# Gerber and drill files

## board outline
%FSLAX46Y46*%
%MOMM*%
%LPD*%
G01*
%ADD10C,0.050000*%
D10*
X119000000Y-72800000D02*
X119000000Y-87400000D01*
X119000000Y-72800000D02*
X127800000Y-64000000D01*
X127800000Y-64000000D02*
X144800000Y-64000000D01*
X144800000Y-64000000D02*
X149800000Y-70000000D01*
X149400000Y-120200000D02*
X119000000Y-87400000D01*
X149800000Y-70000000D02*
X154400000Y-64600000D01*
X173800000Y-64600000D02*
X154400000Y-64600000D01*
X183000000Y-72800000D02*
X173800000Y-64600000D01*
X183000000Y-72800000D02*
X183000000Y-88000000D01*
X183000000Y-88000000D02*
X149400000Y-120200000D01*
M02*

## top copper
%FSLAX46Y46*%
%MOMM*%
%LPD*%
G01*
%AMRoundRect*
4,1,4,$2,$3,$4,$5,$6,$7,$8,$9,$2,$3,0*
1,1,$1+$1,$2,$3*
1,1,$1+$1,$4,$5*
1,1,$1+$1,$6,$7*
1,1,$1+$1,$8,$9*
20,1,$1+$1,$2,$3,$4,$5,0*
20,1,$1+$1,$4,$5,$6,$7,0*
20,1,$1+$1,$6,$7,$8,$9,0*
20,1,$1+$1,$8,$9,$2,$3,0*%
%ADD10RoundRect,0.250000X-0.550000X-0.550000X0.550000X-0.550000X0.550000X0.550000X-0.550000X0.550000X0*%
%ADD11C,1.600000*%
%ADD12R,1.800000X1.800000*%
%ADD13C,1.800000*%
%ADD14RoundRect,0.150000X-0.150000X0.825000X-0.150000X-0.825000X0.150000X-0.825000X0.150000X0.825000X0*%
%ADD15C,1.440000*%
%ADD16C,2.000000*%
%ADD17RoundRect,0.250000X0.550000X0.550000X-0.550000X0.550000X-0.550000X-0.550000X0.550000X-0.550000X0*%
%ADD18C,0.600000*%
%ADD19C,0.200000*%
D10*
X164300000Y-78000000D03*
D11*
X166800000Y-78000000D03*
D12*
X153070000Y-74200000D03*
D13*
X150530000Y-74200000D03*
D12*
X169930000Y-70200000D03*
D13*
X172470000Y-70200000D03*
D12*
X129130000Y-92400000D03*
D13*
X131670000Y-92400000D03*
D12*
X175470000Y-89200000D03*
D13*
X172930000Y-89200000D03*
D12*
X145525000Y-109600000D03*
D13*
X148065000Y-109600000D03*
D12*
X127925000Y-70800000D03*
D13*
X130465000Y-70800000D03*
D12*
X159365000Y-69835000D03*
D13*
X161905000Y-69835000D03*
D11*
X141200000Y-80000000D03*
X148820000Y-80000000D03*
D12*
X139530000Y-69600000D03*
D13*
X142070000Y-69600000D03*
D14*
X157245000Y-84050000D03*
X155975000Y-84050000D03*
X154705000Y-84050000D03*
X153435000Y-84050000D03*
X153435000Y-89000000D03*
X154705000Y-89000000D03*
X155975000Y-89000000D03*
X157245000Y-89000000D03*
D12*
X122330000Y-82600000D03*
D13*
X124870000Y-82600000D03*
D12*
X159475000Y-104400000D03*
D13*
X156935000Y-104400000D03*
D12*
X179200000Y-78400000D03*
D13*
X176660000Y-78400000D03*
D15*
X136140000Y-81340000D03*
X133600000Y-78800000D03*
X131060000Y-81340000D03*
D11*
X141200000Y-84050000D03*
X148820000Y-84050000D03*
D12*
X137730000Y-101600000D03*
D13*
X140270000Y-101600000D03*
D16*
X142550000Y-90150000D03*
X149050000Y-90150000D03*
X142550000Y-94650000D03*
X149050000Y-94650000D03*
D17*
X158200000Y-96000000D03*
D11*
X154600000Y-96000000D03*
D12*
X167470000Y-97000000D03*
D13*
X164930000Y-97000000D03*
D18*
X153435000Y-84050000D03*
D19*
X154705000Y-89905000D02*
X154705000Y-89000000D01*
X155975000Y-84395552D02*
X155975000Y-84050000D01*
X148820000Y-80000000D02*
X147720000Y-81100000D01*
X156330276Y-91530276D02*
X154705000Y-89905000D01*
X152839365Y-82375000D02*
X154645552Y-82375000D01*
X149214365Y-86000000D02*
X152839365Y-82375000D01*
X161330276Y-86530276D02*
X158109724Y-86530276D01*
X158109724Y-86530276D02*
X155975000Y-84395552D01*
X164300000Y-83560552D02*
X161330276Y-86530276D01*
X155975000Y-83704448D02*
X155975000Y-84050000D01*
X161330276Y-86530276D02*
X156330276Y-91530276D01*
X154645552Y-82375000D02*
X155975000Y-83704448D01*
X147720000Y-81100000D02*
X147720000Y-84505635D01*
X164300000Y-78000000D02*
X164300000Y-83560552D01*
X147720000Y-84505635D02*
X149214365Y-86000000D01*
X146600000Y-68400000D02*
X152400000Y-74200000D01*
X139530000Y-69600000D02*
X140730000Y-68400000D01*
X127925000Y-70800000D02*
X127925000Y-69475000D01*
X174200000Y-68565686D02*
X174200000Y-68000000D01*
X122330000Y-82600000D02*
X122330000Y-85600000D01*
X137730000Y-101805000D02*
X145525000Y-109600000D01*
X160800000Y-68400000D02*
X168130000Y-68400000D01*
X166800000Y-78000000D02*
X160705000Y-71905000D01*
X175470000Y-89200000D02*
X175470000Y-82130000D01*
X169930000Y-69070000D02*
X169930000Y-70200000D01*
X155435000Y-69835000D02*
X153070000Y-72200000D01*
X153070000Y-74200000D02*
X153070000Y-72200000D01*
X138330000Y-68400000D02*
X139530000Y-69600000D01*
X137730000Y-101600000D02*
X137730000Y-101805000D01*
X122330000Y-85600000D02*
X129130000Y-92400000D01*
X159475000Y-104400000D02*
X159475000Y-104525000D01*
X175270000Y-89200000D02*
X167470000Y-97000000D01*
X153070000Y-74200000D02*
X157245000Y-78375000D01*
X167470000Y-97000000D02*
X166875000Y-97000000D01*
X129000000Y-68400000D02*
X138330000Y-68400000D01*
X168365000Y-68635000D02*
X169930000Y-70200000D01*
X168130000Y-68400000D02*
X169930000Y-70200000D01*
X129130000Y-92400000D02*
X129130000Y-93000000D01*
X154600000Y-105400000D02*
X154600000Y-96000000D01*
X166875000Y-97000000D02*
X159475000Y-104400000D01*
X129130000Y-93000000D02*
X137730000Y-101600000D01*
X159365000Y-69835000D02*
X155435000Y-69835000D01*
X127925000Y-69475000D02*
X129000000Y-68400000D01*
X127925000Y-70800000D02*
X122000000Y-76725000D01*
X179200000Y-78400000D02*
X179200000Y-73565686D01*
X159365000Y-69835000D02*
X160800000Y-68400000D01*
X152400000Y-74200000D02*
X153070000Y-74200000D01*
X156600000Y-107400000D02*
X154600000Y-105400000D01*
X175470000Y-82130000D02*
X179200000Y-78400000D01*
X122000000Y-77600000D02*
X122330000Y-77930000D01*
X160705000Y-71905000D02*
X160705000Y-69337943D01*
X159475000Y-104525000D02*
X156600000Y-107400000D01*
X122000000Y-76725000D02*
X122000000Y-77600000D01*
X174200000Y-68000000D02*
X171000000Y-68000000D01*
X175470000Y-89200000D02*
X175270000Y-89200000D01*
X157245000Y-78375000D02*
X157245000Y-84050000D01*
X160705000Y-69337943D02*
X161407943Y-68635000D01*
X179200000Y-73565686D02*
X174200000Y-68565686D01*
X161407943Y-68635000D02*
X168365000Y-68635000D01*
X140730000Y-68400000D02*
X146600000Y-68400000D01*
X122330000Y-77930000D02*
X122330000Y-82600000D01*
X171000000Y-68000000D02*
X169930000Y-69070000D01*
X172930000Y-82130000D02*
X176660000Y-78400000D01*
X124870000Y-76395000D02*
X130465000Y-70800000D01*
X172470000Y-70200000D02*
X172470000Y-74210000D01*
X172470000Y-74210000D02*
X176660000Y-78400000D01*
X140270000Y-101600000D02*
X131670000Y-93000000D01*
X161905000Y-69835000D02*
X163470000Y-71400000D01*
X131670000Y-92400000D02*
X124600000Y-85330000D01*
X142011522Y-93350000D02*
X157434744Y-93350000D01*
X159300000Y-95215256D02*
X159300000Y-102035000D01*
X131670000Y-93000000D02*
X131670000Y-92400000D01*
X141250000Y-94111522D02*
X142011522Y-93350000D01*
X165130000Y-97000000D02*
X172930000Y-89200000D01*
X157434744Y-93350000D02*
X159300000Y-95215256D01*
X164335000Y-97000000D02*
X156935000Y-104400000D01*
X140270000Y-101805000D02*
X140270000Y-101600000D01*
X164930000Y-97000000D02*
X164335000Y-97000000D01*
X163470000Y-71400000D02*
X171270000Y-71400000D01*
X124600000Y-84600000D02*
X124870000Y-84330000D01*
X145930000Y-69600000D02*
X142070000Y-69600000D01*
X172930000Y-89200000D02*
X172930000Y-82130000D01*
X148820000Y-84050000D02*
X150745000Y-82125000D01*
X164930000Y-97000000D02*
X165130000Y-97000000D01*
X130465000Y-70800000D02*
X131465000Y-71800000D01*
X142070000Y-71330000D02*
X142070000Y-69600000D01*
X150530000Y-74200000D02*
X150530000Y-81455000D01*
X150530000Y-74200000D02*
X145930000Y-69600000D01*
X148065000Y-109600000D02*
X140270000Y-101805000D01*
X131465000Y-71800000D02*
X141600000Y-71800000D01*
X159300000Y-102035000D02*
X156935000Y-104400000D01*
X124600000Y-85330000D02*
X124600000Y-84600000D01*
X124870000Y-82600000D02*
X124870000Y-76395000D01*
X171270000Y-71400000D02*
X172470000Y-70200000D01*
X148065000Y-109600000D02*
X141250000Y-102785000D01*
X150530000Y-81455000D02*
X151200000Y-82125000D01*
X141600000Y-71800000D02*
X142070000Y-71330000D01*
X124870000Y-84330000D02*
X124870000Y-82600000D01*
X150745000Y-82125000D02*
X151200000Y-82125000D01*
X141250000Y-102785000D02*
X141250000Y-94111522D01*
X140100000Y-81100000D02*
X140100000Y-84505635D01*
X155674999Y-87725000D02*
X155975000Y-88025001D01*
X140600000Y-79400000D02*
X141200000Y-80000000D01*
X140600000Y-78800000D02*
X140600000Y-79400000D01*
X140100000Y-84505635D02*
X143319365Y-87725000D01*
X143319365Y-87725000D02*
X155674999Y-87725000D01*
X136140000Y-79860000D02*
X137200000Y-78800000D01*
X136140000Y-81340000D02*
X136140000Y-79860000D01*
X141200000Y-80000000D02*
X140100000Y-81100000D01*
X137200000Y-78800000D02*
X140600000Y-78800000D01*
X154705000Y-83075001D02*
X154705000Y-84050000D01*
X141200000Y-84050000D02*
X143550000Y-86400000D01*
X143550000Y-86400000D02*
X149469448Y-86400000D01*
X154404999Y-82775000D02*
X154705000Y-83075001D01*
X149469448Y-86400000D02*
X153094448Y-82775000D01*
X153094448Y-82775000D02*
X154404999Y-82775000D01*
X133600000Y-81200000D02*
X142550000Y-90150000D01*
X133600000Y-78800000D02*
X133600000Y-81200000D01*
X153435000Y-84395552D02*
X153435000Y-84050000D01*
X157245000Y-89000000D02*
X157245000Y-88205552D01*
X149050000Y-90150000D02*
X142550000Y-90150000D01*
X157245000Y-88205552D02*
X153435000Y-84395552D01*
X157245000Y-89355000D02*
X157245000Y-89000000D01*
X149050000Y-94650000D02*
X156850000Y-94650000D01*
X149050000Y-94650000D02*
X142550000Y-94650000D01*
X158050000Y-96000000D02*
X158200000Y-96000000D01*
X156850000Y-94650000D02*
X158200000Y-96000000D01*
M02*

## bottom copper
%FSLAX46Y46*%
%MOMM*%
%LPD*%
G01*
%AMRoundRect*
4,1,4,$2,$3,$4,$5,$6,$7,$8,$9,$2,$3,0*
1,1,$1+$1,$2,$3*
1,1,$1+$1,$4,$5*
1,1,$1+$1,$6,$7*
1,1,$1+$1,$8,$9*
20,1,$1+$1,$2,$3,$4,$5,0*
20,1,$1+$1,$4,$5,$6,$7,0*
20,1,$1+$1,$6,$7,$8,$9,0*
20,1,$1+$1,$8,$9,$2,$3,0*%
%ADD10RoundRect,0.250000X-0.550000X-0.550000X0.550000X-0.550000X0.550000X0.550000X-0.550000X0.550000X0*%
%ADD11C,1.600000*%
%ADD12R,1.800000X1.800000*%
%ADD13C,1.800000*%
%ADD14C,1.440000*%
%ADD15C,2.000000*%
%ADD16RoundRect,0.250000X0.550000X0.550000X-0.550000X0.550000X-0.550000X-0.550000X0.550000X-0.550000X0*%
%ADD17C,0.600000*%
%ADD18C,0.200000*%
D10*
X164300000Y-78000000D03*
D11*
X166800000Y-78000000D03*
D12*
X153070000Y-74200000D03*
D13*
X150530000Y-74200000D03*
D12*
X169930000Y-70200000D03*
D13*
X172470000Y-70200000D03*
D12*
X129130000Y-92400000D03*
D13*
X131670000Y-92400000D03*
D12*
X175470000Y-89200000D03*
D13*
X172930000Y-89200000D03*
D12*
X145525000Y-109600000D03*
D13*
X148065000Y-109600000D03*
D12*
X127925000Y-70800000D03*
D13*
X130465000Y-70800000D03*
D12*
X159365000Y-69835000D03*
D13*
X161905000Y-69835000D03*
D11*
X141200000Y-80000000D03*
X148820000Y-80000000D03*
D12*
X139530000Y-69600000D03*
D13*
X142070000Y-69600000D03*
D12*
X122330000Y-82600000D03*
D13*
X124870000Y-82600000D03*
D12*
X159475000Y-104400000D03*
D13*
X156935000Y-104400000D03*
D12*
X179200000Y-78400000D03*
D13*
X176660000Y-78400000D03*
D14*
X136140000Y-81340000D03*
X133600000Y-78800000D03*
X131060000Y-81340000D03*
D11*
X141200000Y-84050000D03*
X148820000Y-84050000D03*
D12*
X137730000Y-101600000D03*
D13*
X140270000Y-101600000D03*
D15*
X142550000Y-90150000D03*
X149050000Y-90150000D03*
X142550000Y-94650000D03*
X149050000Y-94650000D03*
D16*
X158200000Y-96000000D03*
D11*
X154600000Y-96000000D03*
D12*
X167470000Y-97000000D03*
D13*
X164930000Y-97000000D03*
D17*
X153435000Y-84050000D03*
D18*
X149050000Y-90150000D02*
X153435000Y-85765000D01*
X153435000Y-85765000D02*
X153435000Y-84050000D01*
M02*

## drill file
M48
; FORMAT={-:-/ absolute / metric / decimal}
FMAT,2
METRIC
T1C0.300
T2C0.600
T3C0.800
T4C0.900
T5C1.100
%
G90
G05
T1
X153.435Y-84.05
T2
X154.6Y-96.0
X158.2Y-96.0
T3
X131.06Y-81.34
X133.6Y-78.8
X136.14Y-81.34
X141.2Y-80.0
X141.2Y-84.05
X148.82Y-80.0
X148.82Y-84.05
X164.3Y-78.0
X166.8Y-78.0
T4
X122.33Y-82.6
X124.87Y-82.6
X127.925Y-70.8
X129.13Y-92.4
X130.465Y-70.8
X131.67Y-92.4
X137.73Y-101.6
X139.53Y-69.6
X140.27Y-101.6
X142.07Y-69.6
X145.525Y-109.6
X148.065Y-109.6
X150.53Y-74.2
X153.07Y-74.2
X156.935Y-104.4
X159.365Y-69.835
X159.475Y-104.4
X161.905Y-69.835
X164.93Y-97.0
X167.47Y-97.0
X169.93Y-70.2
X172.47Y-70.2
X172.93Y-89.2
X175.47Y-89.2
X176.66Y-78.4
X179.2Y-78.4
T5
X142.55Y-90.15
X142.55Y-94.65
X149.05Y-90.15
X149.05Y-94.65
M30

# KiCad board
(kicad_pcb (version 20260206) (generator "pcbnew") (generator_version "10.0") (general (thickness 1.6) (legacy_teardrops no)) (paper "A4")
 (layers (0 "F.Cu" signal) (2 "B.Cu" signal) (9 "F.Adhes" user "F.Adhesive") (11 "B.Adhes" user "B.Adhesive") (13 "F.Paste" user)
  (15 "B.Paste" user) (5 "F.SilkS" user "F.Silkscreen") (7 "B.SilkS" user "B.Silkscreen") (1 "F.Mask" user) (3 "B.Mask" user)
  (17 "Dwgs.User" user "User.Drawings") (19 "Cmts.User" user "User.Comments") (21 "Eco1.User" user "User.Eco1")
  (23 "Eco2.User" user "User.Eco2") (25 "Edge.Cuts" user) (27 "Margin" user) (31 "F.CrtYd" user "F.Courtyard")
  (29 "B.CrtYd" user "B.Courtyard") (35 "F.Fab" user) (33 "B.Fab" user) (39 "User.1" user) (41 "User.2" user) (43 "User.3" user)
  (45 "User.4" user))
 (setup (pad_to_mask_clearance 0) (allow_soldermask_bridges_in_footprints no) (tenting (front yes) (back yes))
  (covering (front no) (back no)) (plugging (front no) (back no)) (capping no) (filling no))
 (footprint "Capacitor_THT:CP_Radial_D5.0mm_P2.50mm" (layer "F.Cu") (at 164.3 78)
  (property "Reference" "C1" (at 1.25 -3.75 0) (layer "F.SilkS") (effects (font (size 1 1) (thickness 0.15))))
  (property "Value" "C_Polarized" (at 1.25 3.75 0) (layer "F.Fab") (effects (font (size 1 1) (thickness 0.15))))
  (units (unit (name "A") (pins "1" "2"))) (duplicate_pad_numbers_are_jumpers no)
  (pad "1" thru_hole roundrect (at 0 0) (size 1.6 1.6) (drill 0.8) (layers "*.Cu" "*.Mask") (remove_unused_layers no)
   (roundrect_rratio 0.15625) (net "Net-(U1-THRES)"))
  (pad "2" thru_hole circle (at 2.5 0) (size 1.6 1.6) (drill 0.8) (layers "*.Cu" "*.Mask") (remove_unused_layers no) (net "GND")))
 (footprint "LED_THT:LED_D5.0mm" (layer "F.Cu") (at 153.07 74.2 180)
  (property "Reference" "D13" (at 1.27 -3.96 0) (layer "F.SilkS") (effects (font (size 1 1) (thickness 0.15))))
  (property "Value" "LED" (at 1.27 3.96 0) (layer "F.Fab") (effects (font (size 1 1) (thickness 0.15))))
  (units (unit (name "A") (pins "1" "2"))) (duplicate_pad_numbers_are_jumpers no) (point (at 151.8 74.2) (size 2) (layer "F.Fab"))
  (pad "1" thru_hole rect (at 0 0 180) (size 1.8 1.8) (drill 0.9) (layers "*.Cu" "*.Mask") (remove_unused_layers no) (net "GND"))
  (pad "2" thru_hole circle (at 2.54 0 180) (size 1.8 1.8) (drill 0.9) (layers "*.Cu" "*.Mask") (remove_unused_layers no) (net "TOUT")))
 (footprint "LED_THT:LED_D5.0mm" (layer "F.Cu") (at 169.93 70.2)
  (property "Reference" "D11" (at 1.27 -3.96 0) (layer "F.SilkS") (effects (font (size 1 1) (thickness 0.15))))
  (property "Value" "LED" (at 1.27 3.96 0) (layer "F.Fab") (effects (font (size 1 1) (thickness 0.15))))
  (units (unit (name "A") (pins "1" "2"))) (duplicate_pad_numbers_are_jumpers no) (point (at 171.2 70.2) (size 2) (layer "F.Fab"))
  (pad "1" thru_hole rect (at 0 0) (size 1.8 1.8) (drill 0.9) (layers "*.Cu" "*.Mask") (remove_unused_layers no) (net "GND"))
  (pad "2" thru_hole circle (at 2.54 0) (size 1.8 1.8) (drill 0.9) (layers "*.Cu" "*.Mask") (remove_unused_layers no) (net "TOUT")))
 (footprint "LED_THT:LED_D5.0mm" (layer "F.Cu") (at 129.13 92.4)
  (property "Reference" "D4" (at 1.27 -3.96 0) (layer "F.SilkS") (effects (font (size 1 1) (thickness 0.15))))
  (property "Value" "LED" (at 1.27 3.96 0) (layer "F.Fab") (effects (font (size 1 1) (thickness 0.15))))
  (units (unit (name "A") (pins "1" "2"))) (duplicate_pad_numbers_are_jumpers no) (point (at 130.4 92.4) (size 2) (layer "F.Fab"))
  (pad "1" thru_hole rect (at 0 0) (size 1.8 1.8) (drill 0.9) (layers "*.Cu" "*.Mask") (remove_unused_layers no) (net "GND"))
  (pad "2" thru_hole circle (at 2.54 0) (size 1.8 1.8) (drill 0.9) (layers "*.Cu" "*.Mask") (remove_unused_layers no) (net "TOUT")))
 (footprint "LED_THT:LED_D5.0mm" (layer "F.Cu") (at 175.47 89.2 180)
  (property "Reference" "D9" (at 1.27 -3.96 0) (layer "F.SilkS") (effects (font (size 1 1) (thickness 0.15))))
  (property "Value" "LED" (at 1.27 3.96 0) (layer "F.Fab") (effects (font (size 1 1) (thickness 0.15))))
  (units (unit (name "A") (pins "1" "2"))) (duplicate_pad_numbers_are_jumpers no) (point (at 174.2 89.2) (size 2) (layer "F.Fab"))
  (pad "1" thru_hole rect (at 0 0 180) (size 1.8 1.8) (drill 0.9) (layers "*.Cu" "*.Mask") (remove_unused_layers no) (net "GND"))
  (pad "2" thru_hole circle (at 2.54 0 180) (size 1.8 1.8) (drill 0.9) (layers "*.Cu" "*.Mask") (remove_unused_layers no) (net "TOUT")))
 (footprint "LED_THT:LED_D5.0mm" (layer "F.Cu") (at 145.525 109.6)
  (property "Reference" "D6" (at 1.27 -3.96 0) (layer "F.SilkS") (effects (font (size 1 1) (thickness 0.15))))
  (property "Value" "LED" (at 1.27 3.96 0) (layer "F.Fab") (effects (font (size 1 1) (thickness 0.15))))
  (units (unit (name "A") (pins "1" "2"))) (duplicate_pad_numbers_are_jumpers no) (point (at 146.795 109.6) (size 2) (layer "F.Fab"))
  (pad "1" thru_hole rect (at 0 0) (size 1.8 1.8) (drill 0.9) (layers "*.Cu" "*.Mask") (remove_unused_layers no) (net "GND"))
  (pad "2" thru_hole circle (at 2.54 0) (size 1.8 1.8) (drill 0.9) (layers "*.Cu" "*.Mask") (remove_unused_layers no) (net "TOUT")))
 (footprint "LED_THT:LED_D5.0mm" (layer "F.Cu") (at 127.925 70.8)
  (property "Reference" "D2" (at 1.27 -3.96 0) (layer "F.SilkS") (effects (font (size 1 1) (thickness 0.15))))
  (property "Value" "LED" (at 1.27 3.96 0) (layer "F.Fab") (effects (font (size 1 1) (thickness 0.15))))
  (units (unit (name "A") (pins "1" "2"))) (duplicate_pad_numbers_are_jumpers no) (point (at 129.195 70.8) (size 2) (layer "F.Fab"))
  (pad "1" thru_hole rect (at 0 0) (size 1.8 1.8) (drill 0.9) (layers "*.Cu" "*.Mask") (remove_unused_layers no) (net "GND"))
  (pad "2" thru_hole circle (at 2.54 0) (size 1.8 1.8) (drill 0.9) (layers "*.Cu" "*.Mask") (remove_unused_layers no) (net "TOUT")))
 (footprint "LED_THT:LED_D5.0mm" (layer "F.Cu") (at 159.365 69.835)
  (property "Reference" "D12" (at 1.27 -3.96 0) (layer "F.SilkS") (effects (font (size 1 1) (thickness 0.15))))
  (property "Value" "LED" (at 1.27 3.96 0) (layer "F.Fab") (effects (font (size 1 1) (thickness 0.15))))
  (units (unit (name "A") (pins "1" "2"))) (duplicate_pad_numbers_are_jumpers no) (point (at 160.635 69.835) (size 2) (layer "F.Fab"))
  (pad "1" thru_hole rect (at 0 0) (size 1.8 1.8) (drill 0.9) (layers "*.Cu" "*.Mask") (remove_unused_layers no) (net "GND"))
  (pad "2" thru_hole circle (at 2.54 0) (size 1.8 1.8) (drill 0.9) (layers "*.Cu" "*.Mask") (remove_unused_layers no) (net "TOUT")))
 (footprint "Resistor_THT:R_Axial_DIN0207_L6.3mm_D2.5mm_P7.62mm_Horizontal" (layer "F.Cu") (at 141.2 80)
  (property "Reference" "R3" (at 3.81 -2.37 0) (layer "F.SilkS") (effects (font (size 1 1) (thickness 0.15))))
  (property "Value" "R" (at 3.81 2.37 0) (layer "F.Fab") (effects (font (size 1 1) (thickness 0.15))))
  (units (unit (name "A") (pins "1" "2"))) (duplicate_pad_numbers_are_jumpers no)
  (pad "1" thru_hole circle (at 0 0) (size 1.6 1.6) (drill 0.8) (layers "*.Cu" "*.Mask") (remove_unused_layers no) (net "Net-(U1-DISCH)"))
  (pad "2" thru_hole circle (at 7.62 0) (size 1.6 1.6) (drill 0.8) (layers "*.Cu" "*.Mask") (remove_unused_layers no) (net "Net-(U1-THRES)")))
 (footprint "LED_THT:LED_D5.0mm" (layer "F.Cu") (at 139.53 69.6)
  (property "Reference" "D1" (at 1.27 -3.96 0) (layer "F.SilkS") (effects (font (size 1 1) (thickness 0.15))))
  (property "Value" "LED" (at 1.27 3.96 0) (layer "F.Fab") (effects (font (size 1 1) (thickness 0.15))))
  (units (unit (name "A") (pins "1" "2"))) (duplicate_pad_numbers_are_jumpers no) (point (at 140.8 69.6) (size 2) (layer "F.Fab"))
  (pad "1" thru_hole rect (at 0 0) (size 1.8 1.8) (drill 0.9) (layers "*.Cu" "*.Mask") (remove_unused_layers no) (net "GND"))
  (pad "2" thru_hole circle (at 2.54 0) (size 1.8 1.8) (drill 0.9) (layers "*.Cu" "*.Mask") (remove_unused_layers no) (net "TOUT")))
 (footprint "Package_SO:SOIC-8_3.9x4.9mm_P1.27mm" (layer "F.Cu") (at 155.34 86.525 -90)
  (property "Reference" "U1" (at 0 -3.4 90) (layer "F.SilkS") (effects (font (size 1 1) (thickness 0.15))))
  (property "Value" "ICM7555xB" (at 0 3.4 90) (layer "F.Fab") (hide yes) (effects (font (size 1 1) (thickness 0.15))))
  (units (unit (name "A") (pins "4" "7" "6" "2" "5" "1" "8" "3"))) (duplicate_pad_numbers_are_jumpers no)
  (pad "1" smd roundrect (at -2.475 -1.905 270) (size 1.95 0.6) (layers "F.Cu" "F.Mask" "F.Paste") (roundrect_rratio 0.25) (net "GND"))
  (pad "2" smd roundrect (at -2.475 -0.635 270) (size 1.95 0.6) (layers "F.Cu" "F.Mask" "F.Paste") (roundrect_rratio 0.25)
   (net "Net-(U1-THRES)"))
  (pad "3" smd roundrect (at -2.475 0.635 270) (size 1.95 0.6) (layers "F.Cu" "F.Mask" "F.Paste") (roundrect_rratio 0.25)
   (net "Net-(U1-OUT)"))
  (pad "4" smd roundrect (at -2.475 1.905 270) (size 1.95 0.6) (layers "F.Cu" "F.Mask" "F.Paste") (roundrect_rratio 0.25)
   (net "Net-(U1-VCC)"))
  (pad "5" smd roundrect (at 2.475 1.905 270) (size 1.95 0.6) (layers "F.Cu" "F.Mask" "F.Paste") (roundrect_rratio 0.25)
   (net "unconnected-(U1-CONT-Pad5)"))
  (pad "6" smd roundrect (at 2.475 0.635 270) (size 1.95 0.6) (layers "F.Cu" "F.Mask" "F.Paste") (roundrect_rratio 0.25)
   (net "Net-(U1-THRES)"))
  (pad "7" smd roundrect (at 2.475 -0.635 270) (size 1.95 0.6) (layers "F.Cu" "F.Mask" "F.Paste") (roundrect_rratio 0.25)
   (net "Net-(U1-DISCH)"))
  (pad "8" smd roundrect (at 2.475 -1.905 270) (size 1.95 0.6) (layers "F.Cu" "F.Mask" "F.Paste") (roundrect_rratio 0.25)
   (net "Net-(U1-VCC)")))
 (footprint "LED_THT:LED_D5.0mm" (layer "F.Cu") (at 122.33 82.6)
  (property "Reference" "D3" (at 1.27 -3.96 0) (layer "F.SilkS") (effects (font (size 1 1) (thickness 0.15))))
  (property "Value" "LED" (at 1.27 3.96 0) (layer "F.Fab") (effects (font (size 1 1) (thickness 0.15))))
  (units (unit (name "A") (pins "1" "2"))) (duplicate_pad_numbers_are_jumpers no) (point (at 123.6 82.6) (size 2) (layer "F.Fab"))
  (pad "1" thru_hole rect (at 0 0) (size 1.8 1.8) (drill 0.9) (layers "*.Cu" "*.Mask") (remove_unused_layers no) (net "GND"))
  (pad "2" thru_hole circle (at 2.54 0) (size 1.8 1.8) (drill 0.9) (layers "*.Cu" "*.Mask") (remove_unused_layers no) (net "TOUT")))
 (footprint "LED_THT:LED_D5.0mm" (layer "F.Cu") (at 159.475 104.4 180)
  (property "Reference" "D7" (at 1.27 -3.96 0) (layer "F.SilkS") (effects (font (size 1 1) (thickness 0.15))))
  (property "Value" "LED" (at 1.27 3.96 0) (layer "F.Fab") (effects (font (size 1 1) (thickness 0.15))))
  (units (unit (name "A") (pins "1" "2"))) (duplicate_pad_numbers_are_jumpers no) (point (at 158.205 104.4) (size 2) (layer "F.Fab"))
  (pad "1" thru_hole rect (at 0 0 180) (size 1.8 1.8) (drill 0.9) (layers "*.Cu" "*.Mask") (remove_unused_layers no) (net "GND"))
  (pad "2" thru_hole circle (at 2.54 0 180) (size 1.8 1.8) (drill 0.9) (layers "*.Cu" "*.Mask") (remove_unused_layers no) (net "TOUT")))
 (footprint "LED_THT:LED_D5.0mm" (layer "F.Cu") (at 179.2 78.4 180)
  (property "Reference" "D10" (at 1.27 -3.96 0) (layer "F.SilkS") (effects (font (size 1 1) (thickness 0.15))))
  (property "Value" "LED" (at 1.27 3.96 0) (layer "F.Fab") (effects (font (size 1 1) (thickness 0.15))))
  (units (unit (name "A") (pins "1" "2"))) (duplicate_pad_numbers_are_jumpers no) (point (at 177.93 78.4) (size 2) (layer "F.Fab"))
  (pad "1" thru_hole rect (at 0 0 180) (size 1.8 1.8) (drill 0.9) (layers "*.Cu" "*.Mask") (remove_unused_layers no) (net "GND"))
  (pad "2" thru_hole circle (at 2.54 0 180) (size 1.8 1.8) (drill 0.9) (layers "*.Cu" "*.Mask") (remove_unused_layers no) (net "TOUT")))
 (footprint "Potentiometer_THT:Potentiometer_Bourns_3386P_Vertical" (layer "F.Cu") (at 136.14 81.34 90)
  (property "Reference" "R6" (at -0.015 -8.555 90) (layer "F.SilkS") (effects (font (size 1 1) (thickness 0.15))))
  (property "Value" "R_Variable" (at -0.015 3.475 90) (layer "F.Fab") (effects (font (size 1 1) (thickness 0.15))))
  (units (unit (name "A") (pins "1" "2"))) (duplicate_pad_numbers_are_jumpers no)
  (pad "1" thru_hole circle (at 0 0 90) (size 1.44 1.44) (drill 0.8) (layers "*.Cu" "*.Mask") (remove_unused_layers no)
   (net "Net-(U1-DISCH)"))
  (pad "2" thru_hole circle (at 2.54 -2.54 90) (size 1.44 1.44) (drill 0.8) (layers "*.Cu" "*.Mask") (remove_unused_layers no)
   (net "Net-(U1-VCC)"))
  (pad "3" thru_hole circle (at 0 -5.08 90) (size 1.44 1.44) (drill 0.8) (layers "*.Cu" "*.Mask") (remove_unused_layers no)))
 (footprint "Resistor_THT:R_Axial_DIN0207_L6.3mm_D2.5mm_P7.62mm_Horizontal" (layer "F.Cu") (at 141.2 84.05)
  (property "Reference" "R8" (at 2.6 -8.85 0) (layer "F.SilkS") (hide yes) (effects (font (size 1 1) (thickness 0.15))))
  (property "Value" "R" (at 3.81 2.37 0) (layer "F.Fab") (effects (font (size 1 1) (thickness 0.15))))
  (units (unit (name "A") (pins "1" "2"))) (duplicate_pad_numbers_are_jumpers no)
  (pad "1" thru_hole circle (at 0 0) (size 1.6 1.6) (drill 0.8) (layers "*.Cu" "*.Mask") (remove_unused_layers no) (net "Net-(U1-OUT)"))
  (pad "2" thru_hole circle (at 7.62 0) (size 1.6 1.6) (drill 0.8) (layers "*.Cu" "*.Mask") (remove_unused_layers no) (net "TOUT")))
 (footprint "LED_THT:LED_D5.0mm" (layer "F.Cu") (at 137.73 101.6)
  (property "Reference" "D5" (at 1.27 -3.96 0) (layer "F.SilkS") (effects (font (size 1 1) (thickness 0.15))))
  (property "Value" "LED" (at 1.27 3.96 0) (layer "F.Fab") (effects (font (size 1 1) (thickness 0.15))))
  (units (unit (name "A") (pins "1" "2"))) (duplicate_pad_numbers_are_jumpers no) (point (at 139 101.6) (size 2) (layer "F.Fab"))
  (pad "1" thru_hole rect (at 0 0) (size 1.8 1.8) (drill 0.9) (layers "*.Cu" "*.Mask") (remove_unused_layers no) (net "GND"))
  (pad "2" thru_hole circle (at 2.54 0) (size 1.8 1.8) (drill 0.9) (layers "*.Cu" "*.Mask") (remove_unused_layers no) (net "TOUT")))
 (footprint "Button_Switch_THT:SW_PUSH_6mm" (layer "F.Cu") (at 142.55 90.15)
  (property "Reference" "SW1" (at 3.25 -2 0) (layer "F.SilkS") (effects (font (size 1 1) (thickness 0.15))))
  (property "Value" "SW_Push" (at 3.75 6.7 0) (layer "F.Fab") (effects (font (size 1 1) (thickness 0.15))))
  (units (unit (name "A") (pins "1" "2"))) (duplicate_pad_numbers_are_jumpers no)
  (pad "1" thru_hole circle (at 0 0 90) (size 2 2) (drill 1.1) (layers "*.Cu" "*.Mask") (remove_unused_layers no) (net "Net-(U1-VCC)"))
  (pad "1" thru_hole circle (at 6.5 0 90) (size 2 2) (drill 1.1) (layers "*.Cu" "*.Mask") (remove_unused_layers no) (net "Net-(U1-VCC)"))
  (pad "2" thru_hole circle (at 0 4.5 90) (size 2 2) (drill 1.1) (layers "*.Cu" "*.Mask") (remove_unused_layers no) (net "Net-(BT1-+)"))
  (pad "2" thru_hole circle (at 6.5 4.5 90) (size 2 2) (drill 1.1) (layers "*.Cu" "*.Mask") (remove_unused_layers no) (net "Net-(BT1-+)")))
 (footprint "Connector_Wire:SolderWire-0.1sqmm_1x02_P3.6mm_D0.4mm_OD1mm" (layer "F.Cu") (at 158.2 96 180)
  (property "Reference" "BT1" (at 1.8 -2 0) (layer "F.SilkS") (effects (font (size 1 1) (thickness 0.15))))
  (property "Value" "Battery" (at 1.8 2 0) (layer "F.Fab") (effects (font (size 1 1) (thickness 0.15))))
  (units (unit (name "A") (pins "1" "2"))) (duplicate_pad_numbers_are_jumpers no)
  (pad "1" thru_hole roundrect (at 0 0 180) (size 1.6 1.6) (drill 0.6) (layers "*.Cu" "*.Mask") (remove_unused_layers no)
   (roundrect_rratio 0.15625) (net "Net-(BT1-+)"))
  (pad "2" thru_hole circle (at 3.6 0 180) (size 1.6 1.6) (drill 0.6) (layers "*.Cu" "*.Mask") (remove_unused_layers no) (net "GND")))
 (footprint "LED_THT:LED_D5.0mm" (layer "F.Cu") (at 167.47 97 180)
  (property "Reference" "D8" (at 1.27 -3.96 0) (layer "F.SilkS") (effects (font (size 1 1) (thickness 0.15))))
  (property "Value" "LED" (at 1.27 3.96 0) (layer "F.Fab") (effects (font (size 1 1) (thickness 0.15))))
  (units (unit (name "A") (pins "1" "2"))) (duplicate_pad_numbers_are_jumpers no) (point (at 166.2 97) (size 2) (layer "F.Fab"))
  (pad "1" thru_hole rect (at 0 0 180) (size 1.8 1.8) (drill 0.9) (layers "*.Cu" "*.Mask") (remove_unused_layers no) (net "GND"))
  (pad "2" thru_hole circle (at 2.54 0 180) (size 1.8 1.8) (drill 0.9) (layers "*.Cu" "*.Mask") (remove_unused_layers no) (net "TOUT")))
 (gr_line (start 119 72.8) (end 119 87.4) (stroke (width 0.05) (type default)) (layer "Edge.Cuts"))
 (gr_line (start 119 72.8) (end 127.8 64) (stroke (width 0.05) (type default)) (layer "Edge.Cuts"))
 (gr_line (start 127.8 64) (end 144.8 64) (stroke (width 0.05) (type default)) (layer "Edge.Cuts"))
 (gr_line (start 144.8 64) (end 149.8 70) (stroke (width 0.05) (type default)) (layer "Edge.Cuts"))
 (gr_line (start 149.4 120.2) (end 119 87.4) (stroke (width 0.05) (type default)) (layer "Edge.Cuts"))
 (gr_line (start 149.8 70) (end 154.4 64.6) (stroke (width 0.05) (type default)) (layer "Edge.Cuts"))
 (gr_line (start 173.8 64.6) (end 154.4 64.6) (stroke (width 0.05) (type default)) (layer "Edge.Cuts"))
 (gr_line (start 183 72.8) (end 173.8 64.6) (stroke (width 0.05) (type default)) (layer "Edge.Cuts"))
 (gr_line (start 183 72.8) (end 183 88) (stroke (width 0.05) (type default)) (layer "Edge.Cuts"))
 (gr_line (start 183 88) (end 149.4 120.2) (stroke (width 0.05) (type default)) (layer "Edge.Cuts"))
 (segment (start 154.705 89.905) (end 154.705 89) (width 0.2) (layer "F.Cu") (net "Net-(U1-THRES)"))
 (segment (start 155.975 84.395552) (end 155.975 84.05) (width 0.2) (layer "F.Cu") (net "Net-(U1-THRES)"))
 (segment (start 148.82 80) (end 147.72 81.1) (width 0.2) (layer "F.Cu") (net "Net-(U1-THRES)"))
 (segment (start 156.330276 91.530276) (end 154.705 89.905) (width 0.2) (layer "F.Cu") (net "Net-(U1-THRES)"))
 (segment (start 152.839365 82.375) (end 154.645552 82.375) (width 0.2) (layer "F.Cu") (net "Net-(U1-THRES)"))
 (segment (start 149.214365 86) (end 152.839365 82.375) (width 0.2) (layer "F.Cu") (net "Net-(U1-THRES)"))
 (segment (start 161.330276 86.530276) (end 158.109724 86.530276) (width 0.2) (layer "F.Cu") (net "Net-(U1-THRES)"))
 (segment (start 158.109724 86.530276) (end 155.975 84.395552) (width 0.2) (layer "F.Cu") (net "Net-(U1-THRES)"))
 (segment (start 164.3 83.560552) (end 161.330276 86.530276) (width 0.2) (layer "F.Cu") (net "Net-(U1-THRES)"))
 (segment (start 155.975 83.704448) (end 155.975 84.05) (width 0.2) (layer "F.Cu") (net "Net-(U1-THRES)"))
 (segment (start 161.330276 86.530276) (end 156.330276 91.530276) (width 0.2) (layer "F.Cu") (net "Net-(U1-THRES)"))
 (segment (start 154.645552 82.375) (end 155.975 83.704448) (width 0.2) (layer "F.Cu") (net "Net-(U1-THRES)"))
 (segment (start 147.72 81.1) (end 147.72 84.505635) (width 0.2) (layer "F.Cu") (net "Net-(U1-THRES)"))
 (segment (start 164.3 78) (end 164.3 83.560552) (width 0.2) (layer "F.Cu") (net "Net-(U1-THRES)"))
 (segment (start 147.72 84.505635) (end 149.214365 86) (width 0.2) (layer "F.Cu") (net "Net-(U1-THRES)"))
 (segment (start 146.6 68.4) (end 152.4 74.2) (width 0.2) (layer "F.Cu") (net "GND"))
 (segment (start 139.53 69.6) (end 140.73 68.4) (width 0.2) (layer "F.Cu") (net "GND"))
 (segment (start 127.925 70.8) (end 127.925 69.475) (width 0.2) (layer "F.Cu") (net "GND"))
 (segment (start 174.2 68.565686) (end 174.2 68) (width 0.2) (layer "F.Cu") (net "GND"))
 (segment (start 122.33 82.6) (end 122.33 85.6) (width 0.2) (layer "F.Cu") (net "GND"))
 (segment (start 137.73 101.805) (end 145.525 109.6) (width 0.2) (layer "F.Cu") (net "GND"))
 (segment (start 160.8 68.4) (end 168.13 68.4) (width 0.2) (layer "F.Cu") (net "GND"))
 (segment (start 166.8 78) (end 160.705 71.905) (width 0.2) (layer "F.Cu") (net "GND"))
 (segment (start 175.47 89.2) (end 175.47 82.13) (width 0.2) (layer "F.Cu") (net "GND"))
 (segment (start 169.93 69.07) (end 169.93 70.2) (width 0.2) (layer "F.Cu") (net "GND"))
 (segment (start 155.435 69.835) (end 153.07 72.2) (width 0.2) (layer "F.Cu") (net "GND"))
 (segment (start 153.07 74.2) (end 153.07 72.2) (width 0.2) (layer "F.Cu") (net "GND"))
 (segment (start 138.33 68.4) (end 139.53 69.6) (width 0.2) (layer "F.Cu") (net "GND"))
 (segment (start 137.73 101.6) (end 137.73 101.805) (width 0.2) (layer "F.Cu") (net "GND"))
 (segment (start 122.33 85.6) (end 129.13 92.4) (width 0.2) (layer "F.Cu") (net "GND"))
 (segment (start 159.475 104.4) (end 159.475 104.525) (width 0.2) (layer "F.Cu") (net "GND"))
 (segment (start 175.27 89.2) (end 167.47 97) (width 0.2) (layer "F.Cu") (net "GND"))
 (segment (start 153.07 74.2) (end 157.245 78.375) (width 0.2) (layer "F.Cu") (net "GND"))
 (segment (start 167.47 97) (end 166.875 97) (width 0.2) (layer "F.Cu") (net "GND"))
 (segment (start 129 68.4) (end 138.33 68.4) (width 0.2) (layer "F.Cu") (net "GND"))
 (segment (start 168.365 68.635) (end 169.93 70.2) (width 0.2) (layer "F.Cu") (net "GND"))
 (segment (start 168.13 68.4) (end 169.93 70.2) (width 0.2) (layer "F.Cu") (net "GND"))
 (segment (start 129.13 92.4) (end 129.13 93) (width 0.2) (layer "F.Cu") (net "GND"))
 (segment (start 154.6 105.4) (end 154.6 96) (width 0.2) (layer "F.Cu") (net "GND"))
 (segment (start 166.875 97) (end 159.475 104.4) (width 0.2) (layer "F.Cu") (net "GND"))
 (segment (start 129.13 93) (end 137.73 101.6) (width 0.2) (layer "F.Cu") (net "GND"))
 (segment (start 159.365 69.835) (end 155.435 69.835) (width 0.2) (layer "F.Cu") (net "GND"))
 (segment (start 127.925 69.475) (end 129 68.4) (width 0.2) (layer "F.Cu") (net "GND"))
 (segment (start 127.925 70.8) (end 122 76.725) (width 0.2) (layer "F.Cu") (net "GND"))
 (segment (start 179.2 78.4) (end 179.2 73.565686) (width 0.2) (layer "F.Cu") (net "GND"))
 (segment (start 159.365 69.835) (end 160.8 68.4) (width 0.2) (layer "F.Cu") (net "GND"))
 (segment (start 152.4 74.2) (end 153.07 74.2) (width 0.2) (layer "F.Cu") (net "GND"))
 (segment (start 156.6 107.4) (end 154.6 105.4) (width 0.2) (layer "F.Cu") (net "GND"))
 (segment (start 175.47 82.13) (end 179.2 78.4) (width 0.2) (layer "F.Cu") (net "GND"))
 (segment (start 122 77.6) (end 122.33 77.93) (width 0.2) (layer "F.Cu") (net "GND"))
 (segment (start 160.705 71.905) (end 160.705 69.337943) (width 0.2) (layer "F.Cu") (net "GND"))
 (segment (start 159.475 104.525) (end 156.6 107.4) (width 0.2) (layer "F.Cu") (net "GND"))
 (segment (start 122 76.725) (end 122 77.6) (width 0.2) (layer "F.Cu") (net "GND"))
 (segment (start 174.2 68) (end 171 68) (width 0.2) (layer "F.Cu") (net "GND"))
 (segment (start 175.47 89.2) (end 175.27 89.2) (width 0.2) (layer "F.Cu") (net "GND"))
 (segment (start 157.245 78.375) (end 157.245 84.05) (width 0.2) (layer "F.Cu") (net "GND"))
 (segment (start 160.705 69.337943) (end 161.407943 68.635) (width 0.2) (layer "F.Cu") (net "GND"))
 (segment (start 179.2 73.565686) (end 174.2 68.565686) (width 0.2) (layer "F.Cu") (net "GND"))
 (segment (start 161.407943 68.635) (end 168.365 68.635) (width 0.2) (layer "F.Cu") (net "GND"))
 (segment (start 140.73 68.4) (end 146.6 68.4) (width 0.2) (layer "F.Cu") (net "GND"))
 (segment (start 122.33 77.93) (end 122.33 82.6) (width 0.2) (layer "F.Cu") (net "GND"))
 (segment (start 171 68) (end 169.93 69.07) (width 0.2) (layer "F.Cu") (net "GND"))
 (segment (start 172.93 82.13) (end 176.66 78.4) (width 0.2) (layer "F.Cu") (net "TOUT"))
 (segment (start 124.87 76.395) (end 130.465 70.8) (width 0.2) (layer "F.Cu") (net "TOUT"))
 (segment (start 172.47 70.2) (end 172.47 74.21) (width 0.2) (layer "F.Cu") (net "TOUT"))
 (segment (start 172.47 74.21) (end 176.66 78.4) (width 0.2) (layer "F.Cu") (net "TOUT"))
 (segment (start 140.27 101.6) (end 131.67 93) (width 0.2) (layer "F.Cu") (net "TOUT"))
 (segment (start 161.905 69.835) (end 163.47 71.4) (width 0.2) (layer "F.Cu") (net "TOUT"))
 (segment (start 131.67 92.4) (end 124.6 85.33) (width 0.2) (layer "F.Cu") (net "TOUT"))
 (segment (start 142.011522 93.35) (end 157.434744 93.35) (width 0.2) (layer "F.Cu") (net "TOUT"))
 (segment (start 159.3 95.215256) (end 159.3 102.035) (width 0.2) (layer "F.Cu") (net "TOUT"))
 (segment (start 131.67 93) (end 131.67 92.4) (width 0.2) (layer "F.Cu") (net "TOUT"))
 (segment (start 141.25 94.111522) (end 142.011522 93.35) (width 0.2) (layer "F.Cu") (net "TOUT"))
 (segment (start 165.13 97) (end 172.93 89.2) (width 0.2) (layer "F.Cu") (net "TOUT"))
 (segment (start 157.434744 93.35) (end 159.3 95.215256) (width 0.2) (layer "F.Cu") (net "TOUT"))
 (segment (start 164.335 97) (end 156.935 104.4) (width 0.2) (layer "F.Cu") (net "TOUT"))
 (segment (start 140.27 101.805) (end 140.27 101.6) (width 0.2) (layer "F.Cu") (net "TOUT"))
 (segment (start 164.93 97) (end 164.335 97) (width 0.2) (layer "F.Cu") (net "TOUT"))
 (segment (start 163.47 71.4) (end 171.27 71.4) (width 0.2) (layer "F.Cu") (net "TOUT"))
 (segment (start 124.6 84.6) (end 124.87 84.33) (width 0.2) (layer "F.Cu") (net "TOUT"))
 (segment (start 145.93 69.6) (end 142.07 69.6) (width 0.2) (layer "F.Cu") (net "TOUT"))
 (segment (start 172.93 89.2) (end 172.93 82.13) (width 0.2) (layer "F.Cu") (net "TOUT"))
 (segment (start 148.82 84.05) (end 150.745 82.125) (width 0.2) (layer "F.Cu") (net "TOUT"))
 (segment (start 164.93 97) (end 165.13 97) (width 0.2) (layer "F.Cu") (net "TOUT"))
 (segment (start 130.465 70.8) (end 131.465 71.8) (width 0.2) (layer "F.Cu") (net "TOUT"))
 (segment (start 142.07 71.33) (end 142.07 69.6) (width 0.2) (layer "F.Cu") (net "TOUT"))
 (segment (start 150.53 74.2) (end 150.53 81.455) (width 0.2) (layer "F.Cu") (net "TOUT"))
 (segment (start 150.53 74.2) (end 145.93 69.6) (width 0.2) (layer "F.Cu") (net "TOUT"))
 (segment (start 148.065 109.6) (end 140.27 101.805) (width 0.2) (layer "F.Cu") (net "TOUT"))
 (segment (start 131.465 71.8) (end 141.6 71.8) (width 0.2) (layer "F.Cu") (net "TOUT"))
 (segment (start 159.3 102.035) (end 156.935 104.4) (width 0.2) (layer "F.Cu") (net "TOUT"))
 (segment (start 124.6 85.33) (end 124.6 84.6) (width 0.2) (layer "F.Cu") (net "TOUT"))
 (segment (start 124.87 82.6) (end 124.87 76.395) (width 0.2) (layer "F.Cu") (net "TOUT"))
 (segment (start 171.27 71.4) (end 172.47 70.2) (width 0.2) (layer "F.Cu") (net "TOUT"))
 (segment (start 148.065 109.6) (end 141.25 102.785) (width 0.2) (layer "F.Cu") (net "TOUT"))
 (segment (start 150.53 81.455) (end 151.2 82.125) (width 0.2) (layer "F.Cu") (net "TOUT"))
 (segment (start 141.6 71.8) (end 142.07 71.33) (width 0.2) (layer "F.Cu") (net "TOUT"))
 (segment (start 124.87 84.33) (end 124.87 82.6) (width 0.2) (layer "F.Cu") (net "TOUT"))
 (segment (start 150.745 82.125) (end 151.2 82.125) (width 0.2) (layer "F.Cu") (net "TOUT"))
 (segment (start 141.25 102.785) (end 141.25 94.111522) (width 0.2) (layer "F.Cu") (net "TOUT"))
 (segment (start 140.1 81.1) (end 140.1 84.505635) (width 0.2) (layer "F.Cu") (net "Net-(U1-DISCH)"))
 (segment (start 155.674999 87.725) (end 155.975 88.025001) (width 0.2) (layer "F.Cu") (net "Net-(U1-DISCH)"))
 (segment (start 140.6 79.4) (end 141.2 80) (width 0.2) (layer "F.Cu") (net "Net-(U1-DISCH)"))
 (segment (start 140.6 78.8) (end 140.6 79.4) (width 0.2) (layer "F.Cu") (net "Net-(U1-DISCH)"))
 (segment (start 140.1 84.505635) (end 143.319365 87.725) (width 0.2) (layer "F.Cu") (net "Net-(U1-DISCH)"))
 (segment (start 143.319365 87.725) (end 155.674999 87.725) (width 0.2) (layer "F.Cu") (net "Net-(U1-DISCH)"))
 (segment (start 136.14 79.86) (end 137.2 78.8) (width 0.2) (layer "F.Cu") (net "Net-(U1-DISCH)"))
 (segment (start 136.14 81.34) (end 136.14 79.86) (width 0.2) (layer "F.Cu") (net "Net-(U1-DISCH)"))
 (segment (start 141.2 80) (end 140.1 81.1) (width 0.2) (layer "F.Cu") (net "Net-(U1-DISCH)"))
 (segment (start 137.2 78.8) (end 140.6 78.8) (width 0.2) (layer "F.Cu") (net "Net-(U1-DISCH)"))
 (segment (start 154.705 83.075001) (end 154.705 84.05) (width 0.2) (layer "F.Cu") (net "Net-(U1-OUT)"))
 (segment (start 141.2 84.05) (end 143.55 86.4) (width 0.2) (layer "F.Cu") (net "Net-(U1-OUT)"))
 (segment (start 143.55 86.4) (end 149.469448 86.4) (width 0.2) (layer "F.Cu") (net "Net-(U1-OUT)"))
 (segment (start 154.404999 82.775) (end 154.705 83.075001) (width 0.2) (layer "F.Cu") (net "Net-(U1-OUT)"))
 (segment (start 149.469448 86.4) (end 153.094448 82.775) (width 0.2) (layer "F.Cu") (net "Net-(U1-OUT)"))
 (segment (start 153.094448 82.775) (end 154.404999 82.775) (width 0.2) (layer "F.Cu") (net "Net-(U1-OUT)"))
 (segment (start 133.6 81.2) (end 142.55 90.15) (width 0.2) (layer "F.Cu") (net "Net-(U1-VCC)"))
 (segment (start 133.6 78.8) (end 133.6 81.2) (width 0.2) (layer "F.Cu") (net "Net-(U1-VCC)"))
 (segment (start 153.435 84.395552) (end 153.435 84.05) (width 0.2) (layer "F.Cu") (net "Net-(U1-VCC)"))
 (segment (start 157.245 89) (end 157.245 88.205552) (width 0.2) (layer "F.Cu") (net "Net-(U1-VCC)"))
 (segment (start 149.05 90.15) (end 142.55 90.15) (width 0.2) (layer "F.Cu") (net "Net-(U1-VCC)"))
 (segment (start 157.245 88.205552) (end 153.435 84.395552) (width 0.2) (layer "F.Cu") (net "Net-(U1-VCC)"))
 (segment (start 157.245 89.355) (end 157.245 89) (width 0.2) (layer "F.Cu") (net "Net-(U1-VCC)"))
 (via (at 153.435 84.05) (size 0.6) (drill 0.3) (layers "F.Cu" "B.Cu") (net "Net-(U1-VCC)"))
 (segment (start 149.05 90.15) (end 153.435 85.765) (width 0.2) (layer "B.Cu") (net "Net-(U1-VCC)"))
 (segment (start 153.435 85.765) (end 153.435 84.05) (width 0.2) (layer "B.Cu") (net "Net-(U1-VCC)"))
 (segment (start 149.05 94.65) (end 156.85 94.65) (width 0.2) (layer "F.Cu") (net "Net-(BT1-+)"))
 (segment (start 149.05 94.65) (end 142.55 94.65) (width 0.2) (layer "F.Cu") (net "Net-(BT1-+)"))
 (segment (start 158.05 96) (end 158.2 96) (width 0.2) (layer "F.Cu") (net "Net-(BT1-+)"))
 (segment (start 156.85 94.65) (end 158.2 96) (width 0.2) (layer "F.Cu") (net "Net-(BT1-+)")))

